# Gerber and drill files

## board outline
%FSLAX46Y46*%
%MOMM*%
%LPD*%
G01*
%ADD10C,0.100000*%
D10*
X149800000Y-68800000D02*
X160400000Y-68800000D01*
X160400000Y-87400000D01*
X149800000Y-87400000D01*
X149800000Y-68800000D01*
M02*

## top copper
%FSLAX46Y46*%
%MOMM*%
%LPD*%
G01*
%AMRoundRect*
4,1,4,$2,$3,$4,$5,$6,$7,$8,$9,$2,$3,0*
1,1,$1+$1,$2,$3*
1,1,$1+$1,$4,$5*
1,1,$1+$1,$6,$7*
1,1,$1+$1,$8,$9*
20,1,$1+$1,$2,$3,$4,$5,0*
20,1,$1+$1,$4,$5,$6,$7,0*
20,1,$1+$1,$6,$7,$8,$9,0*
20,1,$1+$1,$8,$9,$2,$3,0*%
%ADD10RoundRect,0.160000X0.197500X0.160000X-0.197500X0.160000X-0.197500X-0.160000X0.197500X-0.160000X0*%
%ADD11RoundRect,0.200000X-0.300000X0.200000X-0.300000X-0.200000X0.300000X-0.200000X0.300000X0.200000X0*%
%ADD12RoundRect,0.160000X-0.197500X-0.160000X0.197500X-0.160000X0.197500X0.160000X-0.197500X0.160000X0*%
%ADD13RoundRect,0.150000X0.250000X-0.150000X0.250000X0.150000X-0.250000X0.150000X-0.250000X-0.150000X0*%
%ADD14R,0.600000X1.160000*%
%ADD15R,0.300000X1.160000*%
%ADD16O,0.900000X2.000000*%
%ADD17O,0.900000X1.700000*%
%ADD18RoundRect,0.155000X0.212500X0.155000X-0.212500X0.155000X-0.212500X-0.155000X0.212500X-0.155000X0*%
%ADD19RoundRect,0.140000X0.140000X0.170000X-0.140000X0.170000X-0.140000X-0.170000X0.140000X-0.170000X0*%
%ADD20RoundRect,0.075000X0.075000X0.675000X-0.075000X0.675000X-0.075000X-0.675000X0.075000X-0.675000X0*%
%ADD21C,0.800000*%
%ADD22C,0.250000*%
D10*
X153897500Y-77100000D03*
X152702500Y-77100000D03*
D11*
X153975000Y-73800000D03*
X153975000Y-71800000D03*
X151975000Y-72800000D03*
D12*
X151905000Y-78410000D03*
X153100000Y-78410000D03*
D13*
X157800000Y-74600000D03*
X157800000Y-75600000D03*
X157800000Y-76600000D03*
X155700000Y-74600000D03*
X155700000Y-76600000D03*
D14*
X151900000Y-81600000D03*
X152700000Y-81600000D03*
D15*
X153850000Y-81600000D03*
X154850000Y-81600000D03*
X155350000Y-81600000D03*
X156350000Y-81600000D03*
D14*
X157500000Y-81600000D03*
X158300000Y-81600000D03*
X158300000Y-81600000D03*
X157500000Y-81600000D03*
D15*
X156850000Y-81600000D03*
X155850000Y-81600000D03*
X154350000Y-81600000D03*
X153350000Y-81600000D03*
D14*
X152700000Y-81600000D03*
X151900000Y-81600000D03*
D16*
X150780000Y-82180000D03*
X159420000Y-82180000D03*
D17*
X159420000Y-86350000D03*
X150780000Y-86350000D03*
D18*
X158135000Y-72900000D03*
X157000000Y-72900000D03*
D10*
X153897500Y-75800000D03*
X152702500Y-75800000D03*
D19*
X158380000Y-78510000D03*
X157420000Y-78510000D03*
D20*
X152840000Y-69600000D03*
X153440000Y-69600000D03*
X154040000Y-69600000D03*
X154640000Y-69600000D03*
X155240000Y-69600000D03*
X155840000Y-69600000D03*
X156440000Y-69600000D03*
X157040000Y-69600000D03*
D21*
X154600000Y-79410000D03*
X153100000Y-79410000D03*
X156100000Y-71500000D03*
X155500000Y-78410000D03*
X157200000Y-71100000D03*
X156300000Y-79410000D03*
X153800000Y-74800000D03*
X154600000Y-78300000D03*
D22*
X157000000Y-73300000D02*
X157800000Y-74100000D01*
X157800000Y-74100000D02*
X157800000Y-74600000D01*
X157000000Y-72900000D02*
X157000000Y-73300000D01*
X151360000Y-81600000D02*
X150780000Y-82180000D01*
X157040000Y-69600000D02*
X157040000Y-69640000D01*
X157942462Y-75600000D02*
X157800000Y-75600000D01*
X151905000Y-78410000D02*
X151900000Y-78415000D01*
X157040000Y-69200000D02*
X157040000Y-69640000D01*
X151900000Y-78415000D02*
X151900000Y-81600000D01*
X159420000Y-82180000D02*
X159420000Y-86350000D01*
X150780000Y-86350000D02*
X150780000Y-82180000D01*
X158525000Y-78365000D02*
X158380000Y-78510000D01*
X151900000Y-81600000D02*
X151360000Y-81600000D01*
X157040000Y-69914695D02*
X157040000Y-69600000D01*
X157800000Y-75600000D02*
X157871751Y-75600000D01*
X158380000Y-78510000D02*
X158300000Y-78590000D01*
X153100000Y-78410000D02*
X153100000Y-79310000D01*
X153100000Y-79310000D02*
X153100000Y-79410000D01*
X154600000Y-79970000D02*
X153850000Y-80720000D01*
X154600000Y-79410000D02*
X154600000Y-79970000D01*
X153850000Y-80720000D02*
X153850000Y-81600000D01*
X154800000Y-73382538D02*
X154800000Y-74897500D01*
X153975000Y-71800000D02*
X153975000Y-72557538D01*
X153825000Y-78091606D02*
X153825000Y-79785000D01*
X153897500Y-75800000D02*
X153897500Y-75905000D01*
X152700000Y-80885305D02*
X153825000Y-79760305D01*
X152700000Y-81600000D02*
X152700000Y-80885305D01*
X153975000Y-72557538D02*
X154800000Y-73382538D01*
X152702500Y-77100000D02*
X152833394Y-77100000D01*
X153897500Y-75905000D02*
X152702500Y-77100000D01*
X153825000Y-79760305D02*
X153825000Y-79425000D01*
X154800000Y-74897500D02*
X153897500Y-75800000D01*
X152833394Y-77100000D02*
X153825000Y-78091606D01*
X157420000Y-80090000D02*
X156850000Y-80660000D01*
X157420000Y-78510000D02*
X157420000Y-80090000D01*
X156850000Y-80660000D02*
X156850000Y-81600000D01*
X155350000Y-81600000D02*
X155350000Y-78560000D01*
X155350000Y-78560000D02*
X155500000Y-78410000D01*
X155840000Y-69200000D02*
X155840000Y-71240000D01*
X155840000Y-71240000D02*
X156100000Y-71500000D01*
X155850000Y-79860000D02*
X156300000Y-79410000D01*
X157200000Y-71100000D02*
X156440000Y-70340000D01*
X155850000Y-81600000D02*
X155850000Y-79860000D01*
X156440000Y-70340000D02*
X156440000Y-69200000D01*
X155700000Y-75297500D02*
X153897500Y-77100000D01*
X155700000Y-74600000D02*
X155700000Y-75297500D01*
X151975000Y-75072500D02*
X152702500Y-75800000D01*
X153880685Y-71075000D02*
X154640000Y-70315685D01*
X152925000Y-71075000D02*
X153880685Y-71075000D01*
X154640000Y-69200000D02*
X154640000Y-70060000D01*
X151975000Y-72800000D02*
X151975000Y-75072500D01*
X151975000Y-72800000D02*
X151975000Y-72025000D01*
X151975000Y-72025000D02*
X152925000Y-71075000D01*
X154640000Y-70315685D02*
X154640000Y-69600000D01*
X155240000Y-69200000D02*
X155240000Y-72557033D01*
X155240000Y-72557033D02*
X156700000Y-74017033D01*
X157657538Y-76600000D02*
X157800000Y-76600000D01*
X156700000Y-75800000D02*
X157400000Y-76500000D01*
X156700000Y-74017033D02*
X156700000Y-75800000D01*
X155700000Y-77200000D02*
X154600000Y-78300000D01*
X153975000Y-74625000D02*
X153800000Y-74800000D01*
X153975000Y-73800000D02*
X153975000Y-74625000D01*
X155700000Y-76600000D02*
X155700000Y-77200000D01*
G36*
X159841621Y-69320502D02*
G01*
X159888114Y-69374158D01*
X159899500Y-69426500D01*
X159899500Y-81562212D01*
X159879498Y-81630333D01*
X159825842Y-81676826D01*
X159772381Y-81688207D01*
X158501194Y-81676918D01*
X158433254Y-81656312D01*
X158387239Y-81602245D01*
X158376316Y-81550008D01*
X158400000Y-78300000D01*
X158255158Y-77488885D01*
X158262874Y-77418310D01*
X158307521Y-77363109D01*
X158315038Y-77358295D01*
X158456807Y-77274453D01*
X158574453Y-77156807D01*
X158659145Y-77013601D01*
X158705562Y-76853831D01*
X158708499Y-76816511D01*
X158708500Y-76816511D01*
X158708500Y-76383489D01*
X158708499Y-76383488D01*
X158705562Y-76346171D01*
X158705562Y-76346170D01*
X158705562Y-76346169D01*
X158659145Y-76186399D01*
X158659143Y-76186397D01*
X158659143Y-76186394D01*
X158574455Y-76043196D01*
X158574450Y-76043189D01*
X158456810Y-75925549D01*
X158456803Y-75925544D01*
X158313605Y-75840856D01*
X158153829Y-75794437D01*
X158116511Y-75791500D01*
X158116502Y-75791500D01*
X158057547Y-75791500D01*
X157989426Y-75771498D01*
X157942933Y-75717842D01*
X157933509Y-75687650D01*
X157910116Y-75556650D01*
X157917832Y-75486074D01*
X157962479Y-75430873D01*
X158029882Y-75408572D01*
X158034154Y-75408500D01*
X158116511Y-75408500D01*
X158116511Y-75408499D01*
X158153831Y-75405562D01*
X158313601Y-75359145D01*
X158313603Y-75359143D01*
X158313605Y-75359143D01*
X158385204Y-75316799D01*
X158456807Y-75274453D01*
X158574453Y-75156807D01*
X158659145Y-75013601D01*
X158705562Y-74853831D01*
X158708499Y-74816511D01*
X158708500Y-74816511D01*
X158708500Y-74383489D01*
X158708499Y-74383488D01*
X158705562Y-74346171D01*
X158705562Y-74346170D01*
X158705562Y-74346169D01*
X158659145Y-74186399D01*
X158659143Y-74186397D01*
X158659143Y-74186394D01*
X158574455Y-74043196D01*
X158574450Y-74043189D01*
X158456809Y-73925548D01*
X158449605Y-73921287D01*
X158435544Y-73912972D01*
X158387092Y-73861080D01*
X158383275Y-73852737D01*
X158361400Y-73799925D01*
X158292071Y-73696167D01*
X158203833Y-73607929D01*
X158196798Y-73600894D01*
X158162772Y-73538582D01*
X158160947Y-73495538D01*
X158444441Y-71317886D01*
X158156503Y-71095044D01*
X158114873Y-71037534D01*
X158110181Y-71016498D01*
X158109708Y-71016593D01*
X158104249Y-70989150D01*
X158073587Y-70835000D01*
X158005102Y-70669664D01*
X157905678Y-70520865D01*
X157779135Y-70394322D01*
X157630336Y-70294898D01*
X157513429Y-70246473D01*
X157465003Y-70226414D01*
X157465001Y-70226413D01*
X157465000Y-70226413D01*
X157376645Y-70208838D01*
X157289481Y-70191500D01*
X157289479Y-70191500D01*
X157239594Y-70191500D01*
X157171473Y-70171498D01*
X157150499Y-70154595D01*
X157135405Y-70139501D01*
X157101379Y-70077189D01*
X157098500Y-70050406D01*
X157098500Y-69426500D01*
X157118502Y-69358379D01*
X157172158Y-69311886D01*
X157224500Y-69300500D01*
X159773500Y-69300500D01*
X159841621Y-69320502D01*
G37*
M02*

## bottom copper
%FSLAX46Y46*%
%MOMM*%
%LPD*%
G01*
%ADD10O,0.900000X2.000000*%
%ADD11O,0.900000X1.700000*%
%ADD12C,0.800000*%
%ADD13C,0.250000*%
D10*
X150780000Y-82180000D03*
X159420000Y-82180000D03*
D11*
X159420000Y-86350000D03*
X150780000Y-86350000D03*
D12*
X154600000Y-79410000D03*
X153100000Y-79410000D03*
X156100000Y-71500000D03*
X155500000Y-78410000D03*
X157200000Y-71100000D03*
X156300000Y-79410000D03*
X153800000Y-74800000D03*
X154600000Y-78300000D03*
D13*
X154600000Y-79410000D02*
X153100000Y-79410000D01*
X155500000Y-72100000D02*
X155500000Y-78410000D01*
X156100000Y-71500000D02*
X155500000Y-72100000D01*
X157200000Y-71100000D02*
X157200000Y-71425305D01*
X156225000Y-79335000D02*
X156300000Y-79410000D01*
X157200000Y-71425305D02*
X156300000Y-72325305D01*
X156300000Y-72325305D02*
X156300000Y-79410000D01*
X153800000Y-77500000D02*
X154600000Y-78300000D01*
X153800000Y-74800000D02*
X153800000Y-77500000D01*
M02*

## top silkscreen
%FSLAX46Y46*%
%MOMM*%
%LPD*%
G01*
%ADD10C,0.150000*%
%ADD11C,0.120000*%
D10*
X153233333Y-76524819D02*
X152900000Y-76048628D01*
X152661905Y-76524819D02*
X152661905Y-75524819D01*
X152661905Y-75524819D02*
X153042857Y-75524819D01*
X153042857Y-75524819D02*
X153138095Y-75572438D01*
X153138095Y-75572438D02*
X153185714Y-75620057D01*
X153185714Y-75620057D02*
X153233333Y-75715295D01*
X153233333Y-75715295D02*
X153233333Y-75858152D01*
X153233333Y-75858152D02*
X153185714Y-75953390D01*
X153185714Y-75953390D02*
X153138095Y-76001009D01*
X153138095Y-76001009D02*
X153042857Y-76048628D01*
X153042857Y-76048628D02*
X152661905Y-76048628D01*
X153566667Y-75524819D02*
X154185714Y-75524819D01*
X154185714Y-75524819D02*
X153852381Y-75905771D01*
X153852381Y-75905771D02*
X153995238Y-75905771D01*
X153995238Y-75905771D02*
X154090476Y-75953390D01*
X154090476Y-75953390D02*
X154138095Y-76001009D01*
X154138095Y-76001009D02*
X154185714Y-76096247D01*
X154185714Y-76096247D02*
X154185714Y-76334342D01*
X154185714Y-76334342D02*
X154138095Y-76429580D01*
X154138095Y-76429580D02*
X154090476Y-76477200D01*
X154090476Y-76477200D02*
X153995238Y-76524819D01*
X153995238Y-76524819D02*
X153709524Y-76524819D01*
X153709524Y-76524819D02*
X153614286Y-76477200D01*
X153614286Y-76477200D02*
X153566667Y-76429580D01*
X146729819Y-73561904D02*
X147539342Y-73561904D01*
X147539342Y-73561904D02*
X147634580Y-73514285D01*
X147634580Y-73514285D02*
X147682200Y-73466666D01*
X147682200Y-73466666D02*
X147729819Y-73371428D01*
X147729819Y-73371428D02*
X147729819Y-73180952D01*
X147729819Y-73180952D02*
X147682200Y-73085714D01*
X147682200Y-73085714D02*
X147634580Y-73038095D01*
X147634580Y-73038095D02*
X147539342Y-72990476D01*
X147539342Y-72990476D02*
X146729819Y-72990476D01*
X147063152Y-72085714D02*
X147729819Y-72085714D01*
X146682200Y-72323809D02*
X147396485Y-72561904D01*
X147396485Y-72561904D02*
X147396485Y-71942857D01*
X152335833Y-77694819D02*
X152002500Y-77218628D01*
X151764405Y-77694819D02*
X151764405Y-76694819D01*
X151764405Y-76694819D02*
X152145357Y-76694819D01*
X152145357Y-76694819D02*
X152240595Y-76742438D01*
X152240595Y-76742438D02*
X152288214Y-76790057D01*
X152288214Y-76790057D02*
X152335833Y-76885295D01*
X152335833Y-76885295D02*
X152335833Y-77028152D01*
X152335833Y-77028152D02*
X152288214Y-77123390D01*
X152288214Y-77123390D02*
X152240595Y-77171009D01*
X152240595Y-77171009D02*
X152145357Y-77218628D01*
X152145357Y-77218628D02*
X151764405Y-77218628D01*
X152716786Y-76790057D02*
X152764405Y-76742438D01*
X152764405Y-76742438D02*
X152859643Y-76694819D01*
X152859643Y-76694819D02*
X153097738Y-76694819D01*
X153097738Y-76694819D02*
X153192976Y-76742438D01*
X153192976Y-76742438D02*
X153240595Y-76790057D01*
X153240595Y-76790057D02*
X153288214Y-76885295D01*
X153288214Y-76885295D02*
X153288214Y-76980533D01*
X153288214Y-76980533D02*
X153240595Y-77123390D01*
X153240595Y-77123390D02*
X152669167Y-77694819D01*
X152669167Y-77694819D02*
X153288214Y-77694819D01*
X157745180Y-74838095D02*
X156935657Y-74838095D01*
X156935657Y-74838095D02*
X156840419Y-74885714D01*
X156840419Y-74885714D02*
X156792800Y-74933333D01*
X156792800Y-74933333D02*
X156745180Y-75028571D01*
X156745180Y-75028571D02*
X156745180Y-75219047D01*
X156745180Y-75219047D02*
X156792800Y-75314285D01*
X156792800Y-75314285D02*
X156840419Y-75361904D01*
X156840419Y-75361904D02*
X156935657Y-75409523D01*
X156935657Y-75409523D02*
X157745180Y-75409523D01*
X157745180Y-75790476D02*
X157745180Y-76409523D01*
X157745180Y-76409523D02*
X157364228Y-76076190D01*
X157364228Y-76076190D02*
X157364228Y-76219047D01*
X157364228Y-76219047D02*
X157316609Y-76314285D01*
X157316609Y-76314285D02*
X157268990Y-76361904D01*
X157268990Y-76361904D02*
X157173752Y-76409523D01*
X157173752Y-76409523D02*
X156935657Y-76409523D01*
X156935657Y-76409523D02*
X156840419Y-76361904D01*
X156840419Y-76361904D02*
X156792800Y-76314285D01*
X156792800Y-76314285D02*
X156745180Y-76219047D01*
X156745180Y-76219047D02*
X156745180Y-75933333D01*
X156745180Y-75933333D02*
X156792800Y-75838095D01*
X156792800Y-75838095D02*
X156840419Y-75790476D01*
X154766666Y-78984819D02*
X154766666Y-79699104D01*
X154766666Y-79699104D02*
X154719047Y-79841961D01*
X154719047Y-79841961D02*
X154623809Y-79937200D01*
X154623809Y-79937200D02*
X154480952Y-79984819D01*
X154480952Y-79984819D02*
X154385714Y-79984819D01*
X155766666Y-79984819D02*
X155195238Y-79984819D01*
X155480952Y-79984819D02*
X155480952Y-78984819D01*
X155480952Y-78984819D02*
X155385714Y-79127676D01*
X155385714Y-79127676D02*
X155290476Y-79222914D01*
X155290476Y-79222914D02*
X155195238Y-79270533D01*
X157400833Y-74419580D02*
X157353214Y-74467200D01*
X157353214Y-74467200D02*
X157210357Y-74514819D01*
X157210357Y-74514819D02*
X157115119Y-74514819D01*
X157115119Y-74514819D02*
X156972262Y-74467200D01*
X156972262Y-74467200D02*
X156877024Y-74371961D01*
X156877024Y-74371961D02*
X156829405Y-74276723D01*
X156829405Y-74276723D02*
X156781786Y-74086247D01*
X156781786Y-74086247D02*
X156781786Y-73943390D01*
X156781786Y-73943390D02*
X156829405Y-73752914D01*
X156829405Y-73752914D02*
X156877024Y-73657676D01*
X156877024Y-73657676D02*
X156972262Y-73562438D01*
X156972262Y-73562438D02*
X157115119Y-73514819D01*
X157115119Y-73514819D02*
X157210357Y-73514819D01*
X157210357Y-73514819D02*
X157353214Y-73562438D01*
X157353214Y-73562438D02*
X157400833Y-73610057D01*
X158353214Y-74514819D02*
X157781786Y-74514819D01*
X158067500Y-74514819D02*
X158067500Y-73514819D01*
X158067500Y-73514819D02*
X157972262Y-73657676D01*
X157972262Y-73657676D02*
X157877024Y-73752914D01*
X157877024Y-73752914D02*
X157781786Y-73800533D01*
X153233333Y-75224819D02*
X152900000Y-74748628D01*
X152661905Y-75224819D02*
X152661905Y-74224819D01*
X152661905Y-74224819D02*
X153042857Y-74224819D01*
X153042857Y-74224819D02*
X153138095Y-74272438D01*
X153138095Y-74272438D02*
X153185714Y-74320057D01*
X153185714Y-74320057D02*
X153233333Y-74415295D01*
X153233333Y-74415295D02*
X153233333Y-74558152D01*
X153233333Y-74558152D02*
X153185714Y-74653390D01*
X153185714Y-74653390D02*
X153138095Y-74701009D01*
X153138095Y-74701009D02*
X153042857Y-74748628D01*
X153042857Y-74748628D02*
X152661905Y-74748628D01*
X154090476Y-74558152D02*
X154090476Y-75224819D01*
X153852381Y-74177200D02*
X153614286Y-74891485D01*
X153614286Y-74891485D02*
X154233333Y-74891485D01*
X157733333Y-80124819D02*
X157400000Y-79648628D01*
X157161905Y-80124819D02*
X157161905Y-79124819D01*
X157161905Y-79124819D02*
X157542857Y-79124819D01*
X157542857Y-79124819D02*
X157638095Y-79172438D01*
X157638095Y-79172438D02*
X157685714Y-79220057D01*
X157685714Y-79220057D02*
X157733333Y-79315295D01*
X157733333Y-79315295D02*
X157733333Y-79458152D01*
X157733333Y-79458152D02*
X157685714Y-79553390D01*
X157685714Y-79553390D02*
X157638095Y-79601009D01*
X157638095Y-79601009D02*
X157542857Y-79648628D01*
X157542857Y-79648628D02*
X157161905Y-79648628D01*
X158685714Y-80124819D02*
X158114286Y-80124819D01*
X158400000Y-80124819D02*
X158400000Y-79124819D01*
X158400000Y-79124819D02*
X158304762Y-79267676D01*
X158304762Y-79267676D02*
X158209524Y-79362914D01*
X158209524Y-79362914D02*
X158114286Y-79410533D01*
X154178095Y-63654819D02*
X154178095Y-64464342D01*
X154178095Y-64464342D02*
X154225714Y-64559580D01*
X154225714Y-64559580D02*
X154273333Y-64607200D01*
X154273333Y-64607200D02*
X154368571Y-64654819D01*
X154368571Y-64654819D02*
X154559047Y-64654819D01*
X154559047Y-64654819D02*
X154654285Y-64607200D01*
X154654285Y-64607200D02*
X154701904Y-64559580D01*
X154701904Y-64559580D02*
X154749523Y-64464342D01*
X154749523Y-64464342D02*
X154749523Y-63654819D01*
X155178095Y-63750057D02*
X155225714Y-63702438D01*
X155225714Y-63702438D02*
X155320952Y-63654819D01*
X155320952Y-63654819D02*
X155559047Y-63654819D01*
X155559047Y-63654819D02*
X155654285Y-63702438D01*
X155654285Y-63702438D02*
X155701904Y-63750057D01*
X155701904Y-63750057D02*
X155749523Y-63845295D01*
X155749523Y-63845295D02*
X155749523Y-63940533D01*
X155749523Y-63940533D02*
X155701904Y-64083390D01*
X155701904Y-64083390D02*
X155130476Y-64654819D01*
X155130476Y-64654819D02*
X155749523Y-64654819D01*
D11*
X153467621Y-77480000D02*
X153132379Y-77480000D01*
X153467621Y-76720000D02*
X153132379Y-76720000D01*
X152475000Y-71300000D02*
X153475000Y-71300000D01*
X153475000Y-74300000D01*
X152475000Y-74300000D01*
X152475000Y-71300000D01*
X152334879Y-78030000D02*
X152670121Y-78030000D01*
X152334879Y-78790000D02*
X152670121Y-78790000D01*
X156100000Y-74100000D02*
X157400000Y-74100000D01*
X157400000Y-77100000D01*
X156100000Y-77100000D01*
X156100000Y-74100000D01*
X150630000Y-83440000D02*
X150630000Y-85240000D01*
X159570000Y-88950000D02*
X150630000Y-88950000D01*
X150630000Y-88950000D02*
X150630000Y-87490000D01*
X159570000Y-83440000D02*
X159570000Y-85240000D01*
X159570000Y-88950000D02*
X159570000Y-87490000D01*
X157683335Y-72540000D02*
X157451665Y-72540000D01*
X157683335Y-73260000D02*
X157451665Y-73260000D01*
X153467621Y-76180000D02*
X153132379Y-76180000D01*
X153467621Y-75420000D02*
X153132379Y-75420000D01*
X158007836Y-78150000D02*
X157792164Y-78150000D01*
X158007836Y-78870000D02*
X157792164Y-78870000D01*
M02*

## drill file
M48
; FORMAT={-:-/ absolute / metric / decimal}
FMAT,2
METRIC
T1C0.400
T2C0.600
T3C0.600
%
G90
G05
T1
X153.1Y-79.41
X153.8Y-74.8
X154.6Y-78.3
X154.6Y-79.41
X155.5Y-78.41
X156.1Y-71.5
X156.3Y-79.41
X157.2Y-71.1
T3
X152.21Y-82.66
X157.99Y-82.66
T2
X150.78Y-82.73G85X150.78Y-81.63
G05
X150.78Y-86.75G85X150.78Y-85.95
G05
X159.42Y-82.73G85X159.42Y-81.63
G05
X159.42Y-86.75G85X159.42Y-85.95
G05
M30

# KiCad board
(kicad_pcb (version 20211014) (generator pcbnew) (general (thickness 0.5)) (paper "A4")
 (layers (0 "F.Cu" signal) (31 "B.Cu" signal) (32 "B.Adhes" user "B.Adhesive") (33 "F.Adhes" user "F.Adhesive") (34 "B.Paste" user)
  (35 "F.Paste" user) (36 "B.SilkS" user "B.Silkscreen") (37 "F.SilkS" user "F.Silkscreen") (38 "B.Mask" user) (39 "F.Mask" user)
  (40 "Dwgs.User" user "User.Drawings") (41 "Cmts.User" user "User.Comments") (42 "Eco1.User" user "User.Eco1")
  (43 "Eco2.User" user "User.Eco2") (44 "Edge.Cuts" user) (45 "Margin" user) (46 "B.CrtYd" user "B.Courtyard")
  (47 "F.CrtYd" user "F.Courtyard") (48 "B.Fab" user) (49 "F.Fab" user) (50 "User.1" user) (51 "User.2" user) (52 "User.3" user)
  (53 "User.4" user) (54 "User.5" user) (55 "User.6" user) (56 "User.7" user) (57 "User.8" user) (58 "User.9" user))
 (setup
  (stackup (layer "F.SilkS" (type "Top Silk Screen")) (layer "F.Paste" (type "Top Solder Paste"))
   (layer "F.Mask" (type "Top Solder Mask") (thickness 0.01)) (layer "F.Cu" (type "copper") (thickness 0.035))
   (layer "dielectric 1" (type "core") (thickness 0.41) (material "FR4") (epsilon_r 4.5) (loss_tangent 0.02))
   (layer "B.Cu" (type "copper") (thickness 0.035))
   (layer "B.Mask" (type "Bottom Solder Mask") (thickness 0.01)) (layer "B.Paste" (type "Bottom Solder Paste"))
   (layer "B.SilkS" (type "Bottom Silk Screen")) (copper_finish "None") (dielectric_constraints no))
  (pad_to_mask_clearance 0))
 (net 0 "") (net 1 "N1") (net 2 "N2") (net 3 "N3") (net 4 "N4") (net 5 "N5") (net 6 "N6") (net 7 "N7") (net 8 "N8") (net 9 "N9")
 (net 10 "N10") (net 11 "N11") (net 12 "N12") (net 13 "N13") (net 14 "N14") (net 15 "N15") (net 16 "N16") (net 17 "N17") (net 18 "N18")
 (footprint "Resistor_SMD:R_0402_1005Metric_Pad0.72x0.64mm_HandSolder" (layer "F.Cu") (at 153.3 77.1 180)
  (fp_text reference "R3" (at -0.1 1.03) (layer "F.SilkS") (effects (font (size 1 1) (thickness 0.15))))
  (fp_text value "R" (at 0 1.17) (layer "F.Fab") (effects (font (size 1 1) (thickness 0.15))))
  (fp_line (start -0.167621 -0.38) (end 0.167621 -0.38) (layer "F.SilkS") (width 0.12))
  (fp_line (start -0.167621 0.38) (end 0.167621 0.38) (layer "F.SilkS") (width 0.12))
  (pad "1" smd roundrect (at -0.5975 0 180) (size 0.715 0.64) (layers "F.Cu" "F.Paste" "F.Mask") (roundrect_rratio 0.25) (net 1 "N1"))
  (pad "2" smd roundrect (at 0.5975 0 180) (size 0.715 0.64) (layers "F.Cu" "F.Paste" "F.Mask") (roundrect_rratio 0.25) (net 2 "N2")))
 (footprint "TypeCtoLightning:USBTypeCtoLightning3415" (layer "F.Cu") (at 147.775 72.8 90)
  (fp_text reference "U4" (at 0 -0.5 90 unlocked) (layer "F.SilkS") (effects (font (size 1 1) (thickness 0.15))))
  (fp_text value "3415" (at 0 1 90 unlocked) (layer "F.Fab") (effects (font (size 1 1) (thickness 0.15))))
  (fp_rect (start -1.5 5.7) (end 1.5 4.7) (layer "F.SilkS") (width 0.12) (fill none))
  (pad "1" smd roundrect (at -1 6.2 270) (size 0.8 1) (layers "F.Cu" "F.Paste" "F.Mask") (roundrect_rratio 0.25) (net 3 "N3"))
  (pad "2" smd roundrect (at 1 6.2 270) (size 0.8 1) (layers "F.Cu" "F.Paste" "F.Mask") (roundrect_rratio 0.25) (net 2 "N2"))
  (pad "3" smd roundrect (at 0 4.2 270) (size 0.8 1) (layers "F.Cu" "F.Paste" "F.Mask") (roundrect_rratio 0.25) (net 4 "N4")))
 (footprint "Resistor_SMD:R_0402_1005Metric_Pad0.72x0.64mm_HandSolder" (layer "F.Cu") (at 152.5025 78.41)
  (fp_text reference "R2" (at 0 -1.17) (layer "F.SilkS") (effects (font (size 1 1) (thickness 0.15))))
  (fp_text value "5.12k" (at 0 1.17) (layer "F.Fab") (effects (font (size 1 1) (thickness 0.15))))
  (fp_line (start -0.167621 -0.38) (end 0.167621 -0.38) (layer "F.SilkS") (width 0.12))
  (fp_line (start -0.167621 0.38) (end 0.167621 0.38) (layer "F.SilkS") (width 0.12))
  (pad "1" smd roundrect (at -0.5975 0) (size 0.715 0.64) (layers "F.Cu" "F.Paste" "F.Mask") (roundrect_rratio 0.25) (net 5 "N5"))
  (pad "2" smd roundrect (at 0.5975 0) (size 0.715 0.64) (layers "F.Cu" "F.Paste" "F.Mask") (roundrect_rratio 0.25) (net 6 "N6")))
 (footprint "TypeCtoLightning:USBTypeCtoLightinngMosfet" (layer "F.Cu") (at 156.7 75.6 -90)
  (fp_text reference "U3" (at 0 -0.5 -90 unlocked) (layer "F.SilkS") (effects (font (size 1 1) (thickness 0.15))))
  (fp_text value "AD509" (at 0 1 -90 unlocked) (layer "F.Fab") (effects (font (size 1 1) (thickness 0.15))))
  (fp_rect (start -1.5 -0.7) (end 1.5 0.6) (layer "F.SilkS") (width 0.12) (fill none))
  (pad "1" smd roundrect (at -1 -1.1 90) (size 0.6 0.8) (layers "F.Cu" "F.Paste" "F.Mask") (roundrect_rratio 0.25) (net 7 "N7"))
  (pad "2" smd roundrect (at 0 -1.1 90) (size 0.6 0.8) (layers "F.Cu" "F.Paste" "F.Mask") (roundrect_rratio 0.25) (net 5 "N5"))
  (pad "3" smd roundrect (at 1 -1.1 90) (size 0.6 0.8) (layers "F.Cu" "F.Paste" "F.Mask") (roundrect_rratio 0.25) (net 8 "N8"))
  (pad "4" smd roundrect (at -1 1 90) (size 0.6 0.8) (layers "F.Cu" "F.Paste" "F.Mask") (roundrect_rratio 0.25) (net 1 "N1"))
  (pad "6" smd roundrect (at 1 1 90) (size 0.6 0.8) (layers "F.Cu" "F.Paste" "F.Mask") (roundrect_rratio 0.25) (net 3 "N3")))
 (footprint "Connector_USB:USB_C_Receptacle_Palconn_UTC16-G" (layer "F.Cu") (at 155.1 84.11)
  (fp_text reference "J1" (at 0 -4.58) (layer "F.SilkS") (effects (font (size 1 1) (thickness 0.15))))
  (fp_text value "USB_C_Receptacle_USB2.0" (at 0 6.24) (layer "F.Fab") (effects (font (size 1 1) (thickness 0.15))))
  (fp_line (start -4.47 -0.67) (end -4.47 1.13) (layer "F.SilkS") (width 0.12))
  (fp_line (start 4.47 4.84) (end -4.47 4.84) (layer "F.SilkS") (width 0.12))
  (fp_line (start -4.47 4.84) (end -4.47 3.38) (layer "F.SilkS") (width 0.12))
  (fp_line (start 4.47 -0.67) (end 4.47 1.13) (layer "F.SilkS") (width 0.12))
  (fp_line (start 4.47 4.84) (end 4.47 3.38) (layer "F.SilkS") (width 0.12))
  (pad "" np_thru_hole circle (at -2.89 -1.45 180) (size 0.6 0.6) (drill 0.6) (layers *.Cu *.Mask))
  (pad "" np_thru_hole circle (at 2.89 -1.45 180) (size 0.6 0.6) (drill 0.6) (layers *.Cu *.Mask))
  (pad "A1" smd rect (at -3.2 -2.51) (size 0.6 1.16) (layers "F.Cu" "F.Paste" "F.Mask") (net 5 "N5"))
  (pad "A4" smd rect (at -2.4 -2.51) (size 0.6 1.16) (layers "F.Cu" "F.Paste" "F.Mask") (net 2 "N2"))
  (pad "A5" smd rect (at -1.25 -2.51 180) (size 0.3 1.16) (layers "F.Cu" "F.Paste" "F.Mask") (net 6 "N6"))
  (pad "A6" smd rect (at -0.25 -2.51 180) (size 0.3 1.16) (layers "F.Cu" "F.Paste" "F.Mask") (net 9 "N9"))
  (pad "A7" smd rect (at 0.25 -2.51 180) (size 0.3 1.16) (layers "F.Cu" "F.Paste" "F.Mask") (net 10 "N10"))
  (pad "A8" smd rect (at 1.25 -2.51 180) (size 0.3 1.16) (layers "F.Cu" "F.Paste" "F.Mask") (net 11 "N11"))
  (pad "A9" smd rect (at 2.4 -2.51) (size 0.6 1.16) (layers "F.Cu" "F.Paste" "F.Mask") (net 2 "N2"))
  (pad "A12" smd rect (at 3.2 -2.51) (size 0.6 1.16) (layers "F.Cu" "F.Paste" "F.Mask") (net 5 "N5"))
  (pad "B1" smd rect (at 3.2 -2.51) (size 0.6 1.16) (layers "F.Cu" "F.Paste" "F.Mask") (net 5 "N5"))
  (pad "B4" smd rect (at 2.4 -2.51) (size 0.6 1.16) (layers "F.Cu" "F.Paste" "F.Mask") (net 2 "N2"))
  (pad "B5" smd rect (at 1.75 -2.51 180) (size 0.3 1.16) (layers "F.Cu" "F.Paste" "F.Mask") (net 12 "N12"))
  (pad "B6" smd rect (at 0.75 -2.51 180) (size 0.3 1.16) (layers "F.Cu" "F.Paste" "F.Mask") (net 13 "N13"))
  (pad "B7" smd rect (at -0.75 -2.51 180) (size 0.3 1.16) (layers "F.Cu" "F.Paste" "F.Mask") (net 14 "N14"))
  (pad "B8" smd rect (at -1.75 -2.51 180) (size 0.3 1.16) (layers "F.Cu" "F.Paste" "F.Mask") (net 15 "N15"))
  (pad "B9" smd rect (at -2.4 -2.51) (size 0.6 1.16) (layers "F.Cu" "F.Paste" "F.Mask") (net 2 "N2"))
  (pad "B12" smd rect (at -3.2 -2.51) (size 0.6 1.16) (layers "F.Cu" "F.Paste" "F.Mask") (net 5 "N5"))
  (pad "S1" thru_hole oval (at -4.32 -1.93 90) (size 2 0.9) (drill oval 1.7 0.6) (layers *.Cu *.Mask) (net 5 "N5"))
  (pad "S1" thru_hole oval (at 4.32 -1.93 90) (size 2 0.9) (drill oval 1.7 0.6) (layers *.Cu *.Mask) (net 5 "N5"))
  (pad "S1" thru_hole oval (at 4.32 2.24 90) (size 1.7 0.9) (drill oval 1.4 0.6) (layers *.Cu *.Mask) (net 5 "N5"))
  (pad "S1" thru_hole oval (at -4.32 2.24 90) (size 1.7 0.9) (drill oval 1.4 0.6) (layers *.Cu *.Mask) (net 5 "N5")))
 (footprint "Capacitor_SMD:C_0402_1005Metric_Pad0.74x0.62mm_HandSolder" (layer "F.Cu") (at 157.5675 72.9 180)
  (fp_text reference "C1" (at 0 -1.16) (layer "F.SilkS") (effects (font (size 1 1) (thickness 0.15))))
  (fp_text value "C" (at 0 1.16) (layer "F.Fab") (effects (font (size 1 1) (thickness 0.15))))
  (fp_line (start -0.115835 0.36) (end 0.115835 0.36) (layer "F.SilkS") (width 0.12))
  (fp_line (start -0.115835 -0.36) (end 0.115835 -0.36) (layer "F.SilkS") (width 0.12))
  (pad "1" smd roundrect (at -0.5675 0 180) (size 0.735 0.62) (layers "F.Cu" "F.Paste" "F.Mask") (roundrect_rratio 0.25) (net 5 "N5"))
  (pad "2" smd roundrect (at 0.5675 0 180) (size 0.735 0.62) (layers "F.Cu" "F.Paste" "F.Mask") (roundrect_rratio 0.25) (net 7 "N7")))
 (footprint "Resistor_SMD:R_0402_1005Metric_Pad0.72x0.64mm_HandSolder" (layer "F.Cu") (at 153.3 75.8 180)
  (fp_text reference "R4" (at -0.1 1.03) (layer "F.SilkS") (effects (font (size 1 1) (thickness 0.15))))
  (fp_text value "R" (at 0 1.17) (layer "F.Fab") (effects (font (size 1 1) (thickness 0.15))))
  (fp_line (start -0.167621 -0.38) (end 0.167621 -0.38) (layer "F.SilkS") (width 0.12))
  (fp_line (start -0.167621 0.38) (end 0.167621 0.38) (layer "F.SilkS") (width 0.12))
  (pad "1" smd roundrect (at -0.5975 0 180) (size 0.715 0.64) (layers "F.Cu" "F.Paste" "F.Mask") (roundrect_rratio 0.25) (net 2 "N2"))
  (pad "2" smd roundrect (at 0.5975 0 180) (size 0.715 0.64) (layers "F.Cu" "F.Paste" "F.Mask") (roundrect_rratio 0.25) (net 4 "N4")))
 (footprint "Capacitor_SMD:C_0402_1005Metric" (layer "F.Cu") (at 157.9 78.51 180)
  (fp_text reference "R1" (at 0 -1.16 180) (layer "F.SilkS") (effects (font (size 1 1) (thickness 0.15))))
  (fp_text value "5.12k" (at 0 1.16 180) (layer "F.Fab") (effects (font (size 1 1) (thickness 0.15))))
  (fp_line (start -0.107836 0.36) (end 0.107836 0.36) (layer "F.SilkS") (width 0.12))
  (fp_line (start -0.107836 -0.36) (end 0.107836 -0.36) (layer "F.SilkS") (width 0.12))
  (pad "1" smd roundrect (at -0.48 0 180) (size 0.56 0.62) (layers "F.Cu" "F.Paste" "F.Mask") (roundrect_rratio 0.25) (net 5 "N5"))
  (pad "2" smd roundrect (at 0.48 0 180) (size 0.56 0.62) (layers "F.Cu" "F.Paste" "F.Mask") (roundrect_rratio 0.25) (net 12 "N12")))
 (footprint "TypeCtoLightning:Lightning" (layer "F.Cu") (at 154.94 64.7)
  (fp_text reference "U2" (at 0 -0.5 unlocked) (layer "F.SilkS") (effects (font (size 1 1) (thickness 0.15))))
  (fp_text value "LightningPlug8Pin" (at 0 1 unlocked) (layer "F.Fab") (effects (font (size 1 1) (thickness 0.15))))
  (pad "1" smd roundrect (at -2.1 4.9 180) (size 0.3 1.5) (layers "F.Cu" "F.Paste" "F.Mask") (roundrect_rratio 0.25) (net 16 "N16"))
  (pad "2" smd roundrect (at -1.5 4.9 180) (size 0.3 1.5) (layers "F.Cu" "F.Paste" "F.Mask") (roundrect_rratio 0.25) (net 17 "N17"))
  (pad "3" smd roundrect (at -0.9 4.9 180) (size 0.3 1.5) (layers "F.Cu" "F.Paste" "F.Mask") (roundrect_rratio 0.25) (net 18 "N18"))
  (pad "4" smd roundrect (at -0.3 4.9 180) (size 0.3 1.5) (layers "F.Cu" "F.Paste" "F.Mask") (roundrect_rratio 0.25) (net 4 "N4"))
  (pad "5" smd roundrect (at 0.3 4.9 180) (size 0.3 1.5) (layers "F.Cu" "F.Paste" "F.Mask") (roundrect_rratio 0.25) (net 8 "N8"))
  (pad "6" smd roundrect (at 0.9 4.9 180) (size 0.3 1.5) (layers "F.Cu" "F.Paste" "F.Mask") (roundrect_rratio 0.25) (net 10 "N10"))
  (pad "7" smd roundrect (at 1.5 4.9 180) (size 0.3 1.5) (layers "F.Cu" "F.Paste" "F.Mask") (roundrect_rratio 0.25) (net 13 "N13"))
  (pad "8" smd roundrect (at 2.1 4.9 180) (size 0.3 1.5) (layers "F.Cu" "F.Paste" "F.Mask") (roundrect_rratio 0.25) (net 5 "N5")))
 (gr_rect (start 149.8 87.4) (end 160.4 68.8) (layer "Edge.Cuts") (width 0.1) (fill none))
 (segment (start 157 73.3) (end 157.8 74.1) (width 0.25) (layer "F.Cu") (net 7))
 (segment (start 157.8 74.1) (end 157.8 74.6) (width 0.25) (layer "F.Cu") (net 7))
 (segment (start 157 72.9) (end 157 73.3) (width 0.25) (layer "F.Cu") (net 7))
 (segment (start 151.36 81.6) (end 150.78 82.18) (width 0.25) (layer "F.Cu") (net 5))
 (segment (start 157.04 69.6) (end 157.04 69.64) (width 0.25) (layer "F.Cu") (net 5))
 (segment (start 157.942462 75.6) (end 157.8 75.6) (width 0.25) (layer "F.Cu") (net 5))
 (segment (start 151.905 78.41) (end 151.9 78.415) (width 0.25) (layer "F.Cu") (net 5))
 (segment (start 157.04 69.2) (end 157.04 69.64) (width 0.25) (layer "F.Cu") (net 5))
 (segment (start 151.9 78.415) (end 151.9 81.6) (width 0.25) (layer "F.Cu") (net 5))
 (segment (start 159.42 82.18) (end 159.42 86.35) (width 0.25) (layer "F.Cu") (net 5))
 (segment (start 150.78 86.35) (end 150.78 82.18) (width 0.25) (layer "F.Cu") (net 5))
 (segment (start 158.525 78.365) (end 158.38 78.51) (width 0.25) (layer "F.Cu") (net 5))
 (segment (start 151.9 81.6) (end 151.36 81.6) (width 0.25) (layer "F.Cu") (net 5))
 (segment (start 157.04 69.914695) (end 157.04 69.6) (width 0.25) (layer "F.Cu") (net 5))
 (segment (start 157.8 75.6) (end 157.871751 75.6) (width 0.25) (layer "F.Cu") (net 5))
 (segment (start 158.38 78.51) (end 158.3 78.59) (width 0.25) (layer "F.Cu") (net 5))
 (segment (start 153.1 78.41) (end 153.1 79.31) (width 0.25) (layer "F.Cu") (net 6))
 (segment (start 153.1 79.31) (end 153.1 79.41) (width 0.25) (layer "F.Cu") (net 6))
 (segment (start 154.6 79.97) (end 153.85 80.72) (width 0.25) (layer "F.Cu") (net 6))
 (segment (start 154.6 79.41) (end 154.6 79.97) (width 0.25) (layer "F.Cu") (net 6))
 (segment (start 153.85 80.72) (end 153.85 81.6) (width 0.25) (layer "F.Cu") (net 6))
 (via (at 154.6 79.41) (size 0.8) (drill 0.4) (layers "F.Cu" "B.Cu") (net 6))
 (via (at 153.1 79.41) (size 0.8) (drill 0.4) (layers "F.Cu" "B.Cu") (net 6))
 (segment (start 154.6 79.41) (end 153.1 79.41) (width 0.25) (layer "B.Cu") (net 6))
 (segment (start 154.8 73.382538) (end 154.8 74.8975) (width 0.25) (layer "F.Cu") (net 2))
 (segment (start 153.975 71.8) (end 153.975 72.557538) (width 0.25) (layer "F.Cu") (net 2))
 (segment (start 153.825 78.091606) (end 153.825 79.785) (width 0.25) (layer "F.Cu") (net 2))
 (segment (start 153.8975 75.8) (end 153.8975 75.905) (width 0.25) (layer "F.Cu") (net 2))
 (segment (start 152.7 80.885305) (end 153.825 79.760305) (width 0.25) (layer "F.Cu") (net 2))
 (segment (start 152.7 81.6) (end 152.7 80.885305) (width 0.25) (layer "F.Cu") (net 2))
 (segment (start 153.975 72.557538) (end 154.8 73.382538) (width 0.25) (layer "F.Cu") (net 2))
 (segment (start 152.7025 77.1) (end 152.833394 77.1) (width 0.25) (layer "F.Cu") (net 2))
 (segment (start 153.8975 75.905) (end 152.7025 77.1) (width 0.25) (layer "F.Cu") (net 2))
 (segment (start 153.825 79.760305) (end 153.825 79.425) (width 0.25) (layer "F.Cu") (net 2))
 (segment (start 154.8 74.8975) (end 153.8975 75.8) (width 0.25) (layer "F.Cu") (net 2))
 (segment (start 152.833394 77.1) (end 153.825 78.091606) (width 0.25) (layer "F.Cu") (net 2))
 (segment (start 157.42 80.09) (end 156.85 80.66) (width 0.25) (layer "F.Cu") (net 12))
 (segment (start 157.42 78.51) (end 157.42 80.09) (width 0.25) (layer "F.Cu") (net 12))
 (segment (start 156.85 80.66) (end 156.85 81.6) (width 0.25) (layer "F.Cu") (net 12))
 (segment (start 155.35 81.6) (end 155.35 78.56) (width 0.25) (layer "F.Cu") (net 10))
 (segment (start 155.35 78.56) (end 155.5 78.41) (width 0.25) (layer "F.Cu") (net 10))
 (segment (start 155.84 69.2) (end 155.84 71.24) (width 0.25) (layer "F.Cu") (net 10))
 (segment (start 155.84 71.24) (end 156.1 71.5) (width 0.25) (layer "F.Cu") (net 10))
 (via (at 156.1 71.5) (size 0.8) (drill 0.4) (layers "F.Cu" "B.Cu") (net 10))
 (via (at 155.5 78.41) (size 0.8) (drill 0.4) (layers "F.Cu" "B.Cu") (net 10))
 (segment (start 155.5 72.1) (end 155.5 78.41) (width 0.25) (layer "B.Cu") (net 10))
 (segment (start 156.1 71.5) (end 155.5 72.1) (width 0.25) (layer "B.Cu") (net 10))
 (segment (start 155.85 79.86) (end 156.3 79.41) (width 0.25) (layer "F.Cu") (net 13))
 (segment (start 157.2 71.1) (end 156.44 70.34) (width 0.25) (layer "F.Cu") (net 13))
 (segment (start 155.85 81.6) (end 155.85 79.86) (width 0.25) (layer "F.Cu") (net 13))
 (segment (start 156.44 70.34) (end 156.44 69.2) (width 0.25) (layer "F.Cu") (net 13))
 (via (at 157.2 71.1) (size 0.8) (drill 0.4) (layers "F.Cu" "B.Cu") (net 13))
 (via (at 156.3 79.41) (size 0.8) (drill 0.4) (layers "F.Cu" "B.Cu") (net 13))
 (segment (start 157.2 71.1) (end 157.2 71.425305) (width 0.25) (layer "B.Cu") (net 13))
 (segment (start 156.225 79.335) (end 156.3 79.41) (width 0.25) (layer "B.Cu") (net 13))
 (segment (start 157.2 71.425305) (end 156.3 72.325305) (width 0.25) (layer "B.Cu") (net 13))
 (segment (start 156.3 72.325305) (end 156.3 79.41) (width 0.25) (layer "B.Cu") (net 13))
 (segment (start 155.7 75.2975) (end 153.8975 77.1) (width 0.25) (layer "F.Cu") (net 1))
 (segment (start 155.7 74.6) (end 155.7 75.2975) (width 0.25) (layer "F.Cu") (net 1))
 (segment (start 151.975 75.0725) (end 152.7025 75.8) (width 0.25) (layer "F.Cu") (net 4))
 (segment (start 153.880685 71.075) (end 154.64 70.315685) (width 0.25) (layer "F.Cu") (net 4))
 (segment (start 152.925 71.075) (end 153.880685 71.075) (width 0.25) (layer "F.Cu") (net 4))
 (segment (start 154.64 69.2) (end 154.64 70.06) (width 0.25) (layer "F.Cu") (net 4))
 (segment (start 151.975 72.8) (end 151.975 75.0725) (width 0.25) (layer "F.Cu") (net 4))
 (segment (start 151.975 72.8) (end 151.975 72.025) (width 0.25) (layer "F.Cu") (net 4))
 (segment (start 151.975 72.025) (end 152.925 71.075) (width 0.25) (layer "F.Cu") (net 4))
 (segment (start 154.64 70.315685) (end 154.64 69.6) (width 0.25) (layer "F.Cu") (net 4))
 (segment (start 155.24 69.2) (end 155.24 72.557033) (width 0.25) (layer "F.Cu") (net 8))
 (segment (start 155.24 72.557033) (end 156.7 74.017033) (width 0.25) (layer "F.Cu") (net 8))
 (segment (start 157.657538 76.6) (end 157.8 76.6) (width 0.25) (layer "F.Cu") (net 8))
 (segment (start 156.7 75.8) (end 157.4 76.5) (width 0.25) (layer "F.Cu") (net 8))
 (segment (start 156.7 74.017033) (end 156.7 75.8) (width 0.25) (layer "F.Cu") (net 8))
 (segment (start 155.7 77.2) (end 154.6 78.3) (width 0.25) (layer "F.Cu") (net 3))
 (segment (start 153.975 74.625) (end 153.8 74.8) (width 0.25) (layer "F.Cu") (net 3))
 (segment (start 153.975 73.8) (end 153.975 74.625) (width 0.25) (layer "F.Cu") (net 3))
 (segment (start 155.7 76.6) (end 155.7 77.2) (width 0.25) (layer "F.Cu") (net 3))
 (via (at 153.8 74.8) (size 0.8) (drill 0.4) (layers "F.Cu" "B.Cu") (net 3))
 (via (at 154.6 78.3) (size 0.8) (drill 0.4) (layers "F.Cu" "B.Cu") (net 3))
 (segment (start 153.8 77.5) (end 154.6 78.3) (width 0.25) (layer "B.Cu") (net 3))
 (segment (start 153.8 74.8) (end 153.8 77.5) (width 0.25) (layer "B.Cu") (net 3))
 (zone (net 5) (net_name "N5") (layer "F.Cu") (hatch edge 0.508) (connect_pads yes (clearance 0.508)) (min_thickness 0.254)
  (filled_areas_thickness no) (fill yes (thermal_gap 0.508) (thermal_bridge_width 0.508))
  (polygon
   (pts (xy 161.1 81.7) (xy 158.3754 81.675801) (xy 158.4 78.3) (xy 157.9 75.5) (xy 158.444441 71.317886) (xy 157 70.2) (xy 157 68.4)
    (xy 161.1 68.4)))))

